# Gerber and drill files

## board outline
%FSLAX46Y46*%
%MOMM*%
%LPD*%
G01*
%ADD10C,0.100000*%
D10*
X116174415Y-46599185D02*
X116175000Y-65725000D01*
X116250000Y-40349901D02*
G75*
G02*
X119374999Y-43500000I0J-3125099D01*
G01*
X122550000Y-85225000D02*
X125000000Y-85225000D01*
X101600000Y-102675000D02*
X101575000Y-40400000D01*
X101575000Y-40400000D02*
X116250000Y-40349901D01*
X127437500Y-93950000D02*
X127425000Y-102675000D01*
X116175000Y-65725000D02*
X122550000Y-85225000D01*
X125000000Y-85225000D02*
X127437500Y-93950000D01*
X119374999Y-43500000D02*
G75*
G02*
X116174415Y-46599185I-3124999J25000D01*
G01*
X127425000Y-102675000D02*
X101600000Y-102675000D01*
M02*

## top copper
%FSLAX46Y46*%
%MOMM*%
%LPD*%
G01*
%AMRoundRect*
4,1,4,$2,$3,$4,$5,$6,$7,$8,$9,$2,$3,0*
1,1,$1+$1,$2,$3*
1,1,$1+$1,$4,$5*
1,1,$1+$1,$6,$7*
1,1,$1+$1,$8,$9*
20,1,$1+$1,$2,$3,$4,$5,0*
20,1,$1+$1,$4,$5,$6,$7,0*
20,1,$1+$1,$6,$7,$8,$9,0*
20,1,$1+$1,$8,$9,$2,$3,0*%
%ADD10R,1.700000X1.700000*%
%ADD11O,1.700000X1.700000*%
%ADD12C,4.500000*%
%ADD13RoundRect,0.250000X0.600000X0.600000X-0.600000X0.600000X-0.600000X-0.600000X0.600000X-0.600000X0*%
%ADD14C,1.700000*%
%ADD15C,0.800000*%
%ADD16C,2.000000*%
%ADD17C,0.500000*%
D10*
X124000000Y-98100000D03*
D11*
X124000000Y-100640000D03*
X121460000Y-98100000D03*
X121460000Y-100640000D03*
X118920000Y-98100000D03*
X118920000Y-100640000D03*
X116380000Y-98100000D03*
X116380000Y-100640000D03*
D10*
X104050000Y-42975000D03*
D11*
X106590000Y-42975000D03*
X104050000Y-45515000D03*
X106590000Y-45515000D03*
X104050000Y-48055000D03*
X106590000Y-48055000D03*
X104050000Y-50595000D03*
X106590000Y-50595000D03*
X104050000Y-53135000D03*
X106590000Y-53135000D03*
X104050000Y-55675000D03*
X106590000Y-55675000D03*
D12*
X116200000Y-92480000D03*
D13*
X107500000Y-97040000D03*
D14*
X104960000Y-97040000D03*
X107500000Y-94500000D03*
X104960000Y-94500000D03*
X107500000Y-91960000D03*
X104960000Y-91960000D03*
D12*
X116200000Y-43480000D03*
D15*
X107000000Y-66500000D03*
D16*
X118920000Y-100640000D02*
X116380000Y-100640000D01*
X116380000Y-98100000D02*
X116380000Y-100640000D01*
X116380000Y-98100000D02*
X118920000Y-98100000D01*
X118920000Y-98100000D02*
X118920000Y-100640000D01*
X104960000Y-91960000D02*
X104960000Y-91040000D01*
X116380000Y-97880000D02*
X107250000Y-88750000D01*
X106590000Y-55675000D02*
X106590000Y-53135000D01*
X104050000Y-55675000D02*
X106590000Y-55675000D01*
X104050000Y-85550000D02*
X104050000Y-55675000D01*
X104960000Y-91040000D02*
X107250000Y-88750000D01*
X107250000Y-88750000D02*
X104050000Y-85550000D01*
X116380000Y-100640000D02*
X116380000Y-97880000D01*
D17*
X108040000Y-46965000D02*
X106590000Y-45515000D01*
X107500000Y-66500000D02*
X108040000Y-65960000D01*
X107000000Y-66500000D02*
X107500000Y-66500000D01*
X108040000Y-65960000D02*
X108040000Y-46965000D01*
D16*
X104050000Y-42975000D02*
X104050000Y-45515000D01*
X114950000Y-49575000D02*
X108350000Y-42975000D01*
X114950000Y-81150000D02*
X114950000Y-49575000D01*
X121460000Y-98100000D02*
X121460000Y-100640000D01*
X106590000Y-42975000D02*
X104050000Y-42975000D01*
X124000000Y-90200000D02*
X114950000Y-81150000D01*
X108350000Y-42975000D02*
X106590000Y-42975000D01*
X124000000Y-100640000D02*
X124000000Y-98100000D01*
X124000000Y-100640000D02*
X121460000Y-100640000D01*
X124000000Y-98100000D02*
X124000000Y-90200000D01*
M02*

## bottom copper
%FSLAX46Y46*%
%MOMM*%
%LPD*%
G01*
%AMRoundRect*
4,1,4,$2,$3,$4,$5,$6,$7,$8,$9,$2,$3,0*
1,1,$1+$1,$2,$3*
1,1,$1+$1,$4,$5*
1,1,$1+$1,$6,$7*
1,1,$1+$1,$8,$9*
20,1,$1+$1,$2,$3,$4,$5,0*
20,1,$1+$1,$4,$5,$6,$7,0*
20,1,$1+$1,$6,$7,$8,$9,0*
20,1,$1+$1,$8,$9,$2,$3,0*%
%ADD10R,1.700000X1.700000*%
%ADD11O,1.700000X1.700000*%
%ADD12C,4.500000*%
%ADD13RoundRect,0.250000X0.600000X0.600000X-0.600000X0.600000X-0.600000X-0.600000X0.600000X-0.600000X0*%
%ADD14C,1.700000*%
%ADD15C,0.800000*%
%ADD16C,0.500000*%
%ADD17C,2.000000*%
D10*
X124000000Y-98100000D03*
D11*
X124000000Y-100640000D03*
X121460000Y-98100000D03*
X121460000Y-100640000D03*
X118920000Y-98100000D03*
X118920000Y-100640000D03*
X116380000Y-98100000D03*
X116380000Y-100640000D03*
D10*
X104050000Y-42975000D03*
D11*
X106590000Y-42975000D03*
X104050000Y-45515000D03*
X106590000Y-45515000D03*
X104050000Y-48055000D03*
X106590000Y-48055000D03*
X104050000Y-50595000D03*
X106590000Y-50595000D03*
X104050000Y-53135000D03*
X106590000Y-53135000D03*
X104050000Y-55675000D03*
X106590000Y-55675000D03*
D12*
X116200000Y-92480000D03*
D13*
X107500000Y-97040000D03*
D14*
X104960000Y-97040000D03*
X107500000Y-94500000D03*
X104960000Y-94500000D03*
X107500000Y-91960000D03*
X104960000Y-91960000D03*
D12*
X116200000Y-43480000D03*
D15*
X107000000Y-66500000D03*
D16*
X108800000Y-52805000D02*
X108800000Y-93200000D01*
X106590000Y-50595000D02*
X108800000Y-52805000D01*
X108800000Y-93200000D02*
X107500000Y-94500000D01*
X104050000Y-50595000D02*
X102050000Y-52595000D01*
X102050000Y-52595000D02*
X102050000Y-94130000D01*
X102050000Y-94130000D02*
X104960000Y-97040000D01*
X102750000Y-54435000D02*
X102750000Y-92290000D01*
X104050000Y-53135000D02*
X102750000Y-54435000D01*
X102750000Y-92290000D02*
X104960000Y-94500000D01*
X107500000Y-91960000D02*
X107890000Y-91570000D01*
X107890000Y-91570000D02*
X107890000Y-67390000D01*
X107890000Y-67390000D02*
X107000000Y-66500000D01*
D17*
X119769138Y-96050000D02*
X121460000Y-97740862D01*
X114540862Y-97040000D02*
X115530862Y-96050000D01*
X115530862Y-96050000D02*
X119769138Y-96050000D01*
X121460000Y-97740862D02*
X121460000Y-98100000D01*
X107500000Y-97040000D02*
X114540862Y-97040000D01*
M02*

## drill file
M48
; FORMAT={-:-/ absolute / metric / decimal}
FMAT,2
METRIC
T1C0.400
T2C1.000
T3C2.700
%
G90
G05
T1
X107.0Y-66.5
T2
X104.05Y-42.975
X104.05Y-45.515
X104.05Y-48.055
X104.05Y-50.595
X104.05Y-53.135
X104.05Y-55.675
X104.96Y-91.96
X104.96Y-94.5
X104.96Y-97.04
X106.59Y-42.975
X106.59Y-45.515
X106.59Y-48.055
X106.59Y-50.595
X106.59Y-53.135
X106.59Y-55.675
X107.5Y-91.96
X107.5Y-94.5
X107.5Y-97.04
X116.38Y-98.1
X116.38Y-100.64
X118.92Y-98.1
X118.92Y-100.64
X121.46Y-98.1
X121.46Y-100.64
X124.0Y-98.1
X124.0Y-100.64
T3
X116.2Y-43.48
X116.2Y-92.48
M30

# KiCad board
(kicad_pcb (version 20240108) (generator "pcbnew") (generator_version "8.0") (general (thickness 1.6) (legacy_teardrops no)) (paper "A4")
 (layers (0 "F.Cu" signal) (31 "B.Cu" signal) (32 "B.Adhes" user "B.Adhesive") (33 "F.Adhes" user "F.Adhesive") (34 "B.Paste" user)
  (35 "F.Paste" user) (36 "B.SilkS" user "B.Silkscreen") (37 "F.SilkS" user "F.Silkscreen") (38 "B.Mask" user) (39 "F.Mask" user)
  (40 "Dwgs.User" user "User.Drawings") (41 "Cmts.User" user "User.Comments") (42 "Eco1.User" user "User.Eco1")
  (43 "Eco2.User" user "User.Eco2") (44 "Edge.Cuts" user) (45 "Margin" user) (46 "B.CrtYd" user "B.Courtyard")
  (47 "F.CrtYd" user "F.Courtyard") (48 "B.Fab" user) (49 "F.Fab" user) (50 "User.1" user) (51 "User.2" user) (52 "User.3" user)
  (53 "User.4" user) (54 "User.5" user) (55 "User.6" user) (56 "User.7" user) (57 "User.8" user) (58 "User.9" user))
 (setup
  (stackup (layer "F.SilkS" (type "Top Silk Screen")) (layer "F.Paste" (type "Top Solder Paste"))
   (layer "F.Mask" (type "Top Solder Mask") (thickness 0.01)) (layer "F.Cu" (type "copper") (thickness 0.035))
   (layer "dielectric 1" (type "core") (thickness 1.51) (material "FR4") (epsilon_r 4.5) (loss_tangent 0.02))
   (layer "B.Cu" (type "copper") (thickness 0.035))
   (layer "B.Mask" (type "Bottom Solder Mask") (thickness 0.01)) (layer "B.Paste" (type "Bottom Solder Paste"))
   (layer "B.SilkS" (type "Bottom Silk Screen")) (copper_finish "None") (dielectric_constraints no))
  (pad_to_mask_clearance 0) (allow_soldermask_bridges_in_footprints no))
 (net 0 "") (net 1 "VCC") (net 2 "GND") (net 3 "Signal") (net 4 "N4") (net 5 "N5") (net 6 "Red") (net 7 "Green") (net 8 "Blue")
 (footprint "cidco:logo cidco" (layer "F.Cu") (at 110.5 76.5)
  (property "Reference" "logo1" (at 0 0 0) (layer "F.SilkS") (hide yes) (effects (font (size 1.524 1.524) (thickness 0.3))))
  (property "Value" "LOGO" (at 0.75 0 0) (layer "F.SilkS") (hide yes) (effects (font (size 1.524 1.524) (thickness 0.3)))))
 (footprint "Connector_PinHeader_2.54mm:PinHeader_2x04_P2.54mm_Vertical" (layer "F.Cu") (at 124 98.1 -90)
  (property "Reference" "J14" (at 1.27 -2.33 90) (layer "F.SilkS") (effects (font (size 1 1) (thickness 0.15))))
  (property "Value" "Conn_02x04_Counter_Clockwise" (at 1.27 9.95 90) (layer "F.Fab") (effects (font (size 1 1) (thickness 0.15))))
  (pad "1" thru_hole rect (at 0 0 270) (size 1.7 1.7) (drill 1) (layers "*.Cu" "*.Mask") (remove_unused_layers no) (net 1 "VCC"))
  (pad "2" thru_hole oval (at 2.54 0 270) (size 1.7 1.7) (drill 1) (layers "*.Cu" "*.Mask") (remove_unused_layers no) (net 1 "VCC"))
  (pad "3" thru_hole oval (at 0 2.54 270) (size 1.7 1.7) (drill 1) (layers "*.Cu" "*.Mask") (remove_unused_layers no) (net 1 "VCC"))
  (pad "4" thru_hole oval (at 2.54 2.54 270) (size 1.7 1.7) (drill 1) (layers "*.Cu" "*.Mask") (remove_unused_layers no) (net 1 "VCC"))
  (pad "5" thru_hole oval (at 0 5.08 270) (size 1.7 1.7) (drill 1) (layers "*.Cu" "*.Mask") (remove_unused_layers no) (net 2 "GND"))
  (pad "6" thru_hole oval (at 2.54 5.08 270) (size 1.7 1.7) (drill 1) (layers "*.Cu" "*.Mask") (remove_unused_layers no) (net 2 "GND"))
  (pad "7" thru_hole oval (at 0 7.62 270) (size 1.7 1.7) (drill 1) (layers "*.Cu" "*.Mask") (remove_unused_layers no) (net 2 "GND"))
  (pad "8" thru_hole oval (at 2.54 7.62 270) (size 1.7 1.7) (drill 1) (layers "*.Cu" "*.Mask") (remove_unused_layers no) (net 2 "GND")))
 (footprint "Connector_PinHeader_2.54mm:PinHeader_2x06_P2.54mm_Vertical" (layer "F.Cu") (at 104.05 42.975)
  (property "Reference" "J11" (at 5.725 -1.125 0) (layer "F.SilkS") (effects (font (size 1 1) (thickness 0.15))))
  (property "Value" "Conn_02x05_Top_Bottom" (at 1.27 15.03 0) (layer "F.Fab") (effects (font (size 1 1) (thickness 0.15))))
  (pad "1" thru_hole rect (at 0 0) (size 1.7 1.7) (drill 1) (layers "*.Cu" "*.Mask") (remove_unused_layers no) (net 1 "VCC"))
  (pad "2" thru_hole oval (at 2.54 0) (size 1.7 1.7) (drill 1) (layers "*.Cu" "*.Mask") (remove_unused_layers no) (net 1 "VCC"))
  (pad "3" thru_hole oval (at 0 2.54) (size 1.7 1.7) (drill 1) (layers "*.Cu" "*.Mask") (remove_unused_layers no) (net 1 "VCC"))
  (pad "4" thru_hole oval (at 2.54 2.54) (size 1.7 1.7) (drill 1) (layers "*.Cu" "*.Mask") (remove_unused_layers no) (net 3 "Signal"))
  (pad "5" thru_hole oval (at 0 5.08) (size 1.7 1.7) (drill 1) (layers "*.Cu" "*.Mask") (remove_unused_layers no) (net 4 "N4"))
  (pad "6" thru_hole oval (at 2.54 5.08) (size 1.7 1.7) (drill 1) (layers "*.Cu" "*.Mask") (remove_unused_layers no) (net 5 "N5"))
  (pad "7" thru_hole oval (at 0 7.62) (size 1.7 1.7) (drill 1) (layers "*.Cu" "*.Mask") (remove_unused_layers no) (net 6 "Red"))
  (pad "8" thru_hole oval (at 2.54 7.62) (size 1.7 1.7) (drill 1) (layers "*.Cu" "*.Mask") (remove_unused_layers no) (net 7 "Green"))
  (pad "9" thru_hole oval (at 0 10.16) (size 1.7 1.7) (drill 1) (layers "*.Cu" "*.Mask") (remove_unused_layers no) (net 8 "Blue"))
  (pad "10" thru_hole oval (at 2.54 10.16) (size 1.7 1.7) (drill 1) (layers "*.Cu" "*.Mask") (remove_unused_layers no) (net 2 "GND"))
  (pad "11" thru_hole oval (at 0 12.7) (size 1.7 1.7) (drill 1) (layers "*.Cu" "*.Mask") (remove_unused_layers no) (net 2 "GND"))
  (pad "12" thru_hole oval (at 2.54 12.7) (size 1.7 1.7) (drill 1) (layers "*.Cu" "*.Mask") (remove_unused_layers no) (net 2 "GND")))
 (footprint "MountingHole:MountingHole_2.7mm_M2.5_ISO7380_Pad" (layer "F.Cu") (at 116.2 92.48)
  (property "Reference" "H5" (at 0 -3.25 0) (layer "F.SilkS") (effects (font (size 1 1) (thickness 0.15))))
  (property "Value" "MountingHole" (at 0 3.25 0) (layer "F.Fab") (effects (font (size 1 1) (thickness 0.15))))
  (pad "1" thru_hole circle (at 0 0) (size 4.5 4.5) (drill 2.7) (layers "*.Cu" "*.Mask") (remove_unused_layers no)))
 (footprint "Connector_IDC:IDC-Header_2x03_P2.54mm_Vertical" (layer "F.Cu") (at 107.5 97.04 180)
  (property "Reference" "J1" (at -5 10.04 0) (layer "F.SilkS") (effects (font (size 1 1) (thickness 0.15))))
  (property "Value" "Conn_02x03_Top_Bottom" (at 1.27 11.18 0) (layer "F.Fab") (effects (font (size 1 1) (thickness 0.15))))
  (pad "1" thru_hole roundrect (at 0 0 180) (size 1.7 1.7) (drill 1) (layers "*.Cu" "*.Mask") (remove_unused_layers no)
   (roundrect_rratio 0.147059) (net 1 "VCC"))
  (pad "2" thru_hole circle (at 2.54 0 180) (size 1.7 1.7) (drill 1) (layers "*.Cu" "*.Mask") (remove_unused_layers no) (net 6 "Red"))
  (pad "3" thru_hole circle (at 0 2.54 180) (size 1.7 1.7) (drill 1) (layers "*.Cu" "*.Mask") (remove_unused_layers no) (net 7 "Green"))
  (pad "4" thru_hole circle (at 2.54 2.54 180) (size 1.7 1.7) (drill 1) (layers "*.Cu" "*.Mask") (remove_unused_layers no) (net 8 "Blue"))
  (pad "5" thru_hole circle (at 0 5.08 180) (size 1.7 1.7) (drill 1) (layers "*.Cu" "*.Mask") (remove_unused_layers no) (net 3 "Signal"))
  (pad "6" thru_hole circle (at 2.54 5.08 180) (size 1.7 1.7) (drill 1) (layers "*.Cu" "*.Mask") (remove_unused_layers no) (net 2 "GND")))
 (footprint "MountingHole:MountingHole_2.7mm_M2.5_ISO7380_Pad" (layer "F.Cu") (at 116.2 43.48)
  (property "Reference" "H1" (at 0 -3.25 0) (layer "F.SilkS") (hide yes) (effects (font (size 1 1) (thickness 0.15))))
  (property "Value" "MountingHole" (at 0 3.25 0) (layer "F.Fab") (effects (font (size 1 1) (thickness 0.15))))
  (pad "1" thru_hole circle (at 0 0) (size 4.5 4.5) (drill 2.7) (layers "*.Cu" "*.Mask") (remove_unused_layers no)))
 (gr_line (start 116.174415 46.599185) (end 116.175 65.725) (stroke (width 0.1) (type default)) (layer "Edge.Cuts"))
 (gr_arc (start 116.25 40.349901) (mid 118.4686 41.274078) (end 119.374999 43.5) (stroke (width 0.1) (type default)) (layer "Edge.Cuts"))
 (gr_line (start 122.55 85.225) (end 125 85.225) (stroke (width 0.1) (type default)) (layer "Edge.Cuts"))
 (gr_line (start 101.6 102.675) (end 101.575 40.4) (stroke (width 0.1) (type default)) (layer "Edge.Cuts"))
 (gr_line (start 101.575 40.4) (end 116.25 40.349901) (stroke (width 0.1) (type default)) (layer "Edge.Cuts"))
 (gr_line (start 127.4375 93.95) (end 127.425 102.675) (stroke (width 0.1) (type default)) (layer "Edge.Cuts"))
 (gr_line (start 116.175 65.725) (end 122.55 85.225) (stroke (width 0.1) (type default)) (layer "Edge.Cuts"))
 (gr_line (start 125 85.225) (end 127.4375 93.95) (stroke (width 0.1) (type default)) (layer "Edge.Cuts"))
 (gr_arc (start 119.374999 43.5) (mid 118.423929 45.720056) (end 116.174415 46.599185) (stroke (width 0.1) (type default))
  (layer "Edge.Cuts"))
 (gr_line (start 127.425 102.675) (end 101.6 102.675) (stroke (width 0.1) (type default)) (layer "Edge.Cuts"))
 (segment (start 118.92 100.64) (end 116.38 100.64) (width 2) (layer "F.Cu") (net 2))
 (segment (start 116.38 98.1) (end 116.38 100.64) (width 2) (layer "F.Cu") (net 2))
 (segment (start 116.38 98.1) (end 118.92 98.1) (width 2) (layer "F.Cu") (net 2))
 (segment (start 118.92 98.1) (end 118.92 100.64) (width 2) (layer "F.Cu") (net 2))
 (segment (start 104.96 91.96) (end 104.96 91.04) (width 2) (layer "F.Cu") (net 2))
 (segment (start 116.38 97.88) (end 107.25 88.75) (width 2) (layer "F.Cu") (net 2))
 (segment (start 106.59 55.675) (end 106.59 53.135) (width 2) (layer "F.Cu") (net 2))
 (segment (start 104.05 55.675) (end 106.59 55.675) (width 2) (layer "F.Cu") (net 2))
 (segment (start 104.05 85.55) (end 104.05 55.675) (width 2) (layer "F.Cu") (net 2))
 (segment (start 104.96 91.04) (end 107.25 88.75) (width 2) (layer "F.Cu") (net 2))
 (segment (start 107.25 88.75) (end 104.05 85.55) (width 2) (layer "F.Cu") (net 2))
 (segment (start 116.38 100.64) (end 116.38 97.88) (width 2) (layer "F.Cu") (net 2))
 (segment (start 108.8 52.805) (end 108.8 93.2) (width 0.5) (layer "B.Cu") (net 7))
 (segment (start 106.59 50.595) (end 108.8 52.805) (width 0.5) (layer "B.Cu") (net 7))
 (segment (start 108.8 93.2) (end 107.5 94.5) (width 0.5) (layer "B.Cu") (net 7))
 (segment (start 104.05 50.595) (end 102.05 52.595) (width 0.5) (layer "B.Cu") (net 6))
 (segment (start 102.05 52.595) (end 102.05 94.13) (width 0.5) (layer "B.Cu") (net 6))
 (segment (start 102.05 94.13) (end 104.96 97.04) (width 0.5) (layer "B.Cu") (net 6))
 (segment (start 102.75 54.435) (end 102.75 92.29) (width 0.5) (layer "B.Cu") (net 8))
 (segment (start 104.05 53.135) (end 102.75 54.435) (width 0.5) (layer "B.Cu") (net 8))
 (segment (start 102.75 92.29) (end 104.96 94.5) (width 0.5) (layer "B.Cu") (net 8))
 (segment (start 108.04 46.965) (end 106.59 45.515) (width 0.5) (layer "F.Cu") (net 3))
 (segment (start 107.5 66.5) (end 108.04 65.96) (width 0.5) (layer "F.Cu") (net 3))
 (segment (start 107 66.5) (end 107.5 66.5) (width 0.5) (layer "F.Cu") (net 3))
 (segment (start 108.04 65.96) (end 108.04 46.965) (width 0.5) (layer "F.Cu") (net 3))
 (via (at 107 66.5) (size 0.8) (drill 0.4) (layers "F.Cu" "B.Cu") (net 3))
 (segment (start 107.5 91.96) (end 107.89 91.57) (width 0.5) (layer "B.Cu") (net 3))
 (segment (start 107.89 91.57) (end 107.89 67.39) (width 0.5) (layer "B.Cu") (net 3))
 (segment (start 107.89 67.39) (end 107 66.5) (width 0.5) (layer "B.Cu") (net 3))
 (segment (start 104.05 42.975) (end 104.05 45.515) (width 2) (layer "F.Cu") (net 1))
 (segment (start 114.95 49.575) (end 108.35 42.975) (width 2) (layer "F.Cu") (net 1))
 (segment (start 114.95 81.15) (end 114.95 49.575) (width 2) (layer "F.Cu") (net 1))
 (segment (start 121.46 98.1) (end 121.46 100.64) (width 2) (layer "F.Cu") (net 1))
 (segment (start 106.59 42.975) (end 104.05 42.975) (width 2) (layer "F.Cu") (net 1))
 (segment (start 124 90.2) (end 114.95 81.15) (width 2) (layer "F.Cu") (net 1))
 (segment (start 108.35 42.975) (end 106.59 42.975) (width 2) (layer "F.Cu") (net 1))
 (segment (start 124 100.64) (end 124 98.1) (width 2) (layer "F.Cu") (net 1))
 (segment (start 124 100.64) (end 121.46 100.64) (width 2) (layer "F.Cu") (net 1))
 (segment (start 124 98.1) (end 124 90.2) (width 2) (layer "F.Cu") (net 1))
 (segment (start 119.769138 96.05) (end 121.46 97.740862) (width 2) (layer "B.Cu") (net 1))
 (segment (start 114.540862 97.04) (end 115.530862 96.05) (width 2) (layer "B.Cu") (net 1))
 (segment (start 115.530862 96.05) (end 119.769138 96.05) (width 2) (layer "B.Cu") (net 1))
 (segment (start 121.46 97.740862) (end 121.46 98.1) (width 2) (layer "B.Cu") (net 1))
 (segment (start 107.5 97.04) (end 114.540862 97.04) (width 2) (layer "B.Cu") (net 1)))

